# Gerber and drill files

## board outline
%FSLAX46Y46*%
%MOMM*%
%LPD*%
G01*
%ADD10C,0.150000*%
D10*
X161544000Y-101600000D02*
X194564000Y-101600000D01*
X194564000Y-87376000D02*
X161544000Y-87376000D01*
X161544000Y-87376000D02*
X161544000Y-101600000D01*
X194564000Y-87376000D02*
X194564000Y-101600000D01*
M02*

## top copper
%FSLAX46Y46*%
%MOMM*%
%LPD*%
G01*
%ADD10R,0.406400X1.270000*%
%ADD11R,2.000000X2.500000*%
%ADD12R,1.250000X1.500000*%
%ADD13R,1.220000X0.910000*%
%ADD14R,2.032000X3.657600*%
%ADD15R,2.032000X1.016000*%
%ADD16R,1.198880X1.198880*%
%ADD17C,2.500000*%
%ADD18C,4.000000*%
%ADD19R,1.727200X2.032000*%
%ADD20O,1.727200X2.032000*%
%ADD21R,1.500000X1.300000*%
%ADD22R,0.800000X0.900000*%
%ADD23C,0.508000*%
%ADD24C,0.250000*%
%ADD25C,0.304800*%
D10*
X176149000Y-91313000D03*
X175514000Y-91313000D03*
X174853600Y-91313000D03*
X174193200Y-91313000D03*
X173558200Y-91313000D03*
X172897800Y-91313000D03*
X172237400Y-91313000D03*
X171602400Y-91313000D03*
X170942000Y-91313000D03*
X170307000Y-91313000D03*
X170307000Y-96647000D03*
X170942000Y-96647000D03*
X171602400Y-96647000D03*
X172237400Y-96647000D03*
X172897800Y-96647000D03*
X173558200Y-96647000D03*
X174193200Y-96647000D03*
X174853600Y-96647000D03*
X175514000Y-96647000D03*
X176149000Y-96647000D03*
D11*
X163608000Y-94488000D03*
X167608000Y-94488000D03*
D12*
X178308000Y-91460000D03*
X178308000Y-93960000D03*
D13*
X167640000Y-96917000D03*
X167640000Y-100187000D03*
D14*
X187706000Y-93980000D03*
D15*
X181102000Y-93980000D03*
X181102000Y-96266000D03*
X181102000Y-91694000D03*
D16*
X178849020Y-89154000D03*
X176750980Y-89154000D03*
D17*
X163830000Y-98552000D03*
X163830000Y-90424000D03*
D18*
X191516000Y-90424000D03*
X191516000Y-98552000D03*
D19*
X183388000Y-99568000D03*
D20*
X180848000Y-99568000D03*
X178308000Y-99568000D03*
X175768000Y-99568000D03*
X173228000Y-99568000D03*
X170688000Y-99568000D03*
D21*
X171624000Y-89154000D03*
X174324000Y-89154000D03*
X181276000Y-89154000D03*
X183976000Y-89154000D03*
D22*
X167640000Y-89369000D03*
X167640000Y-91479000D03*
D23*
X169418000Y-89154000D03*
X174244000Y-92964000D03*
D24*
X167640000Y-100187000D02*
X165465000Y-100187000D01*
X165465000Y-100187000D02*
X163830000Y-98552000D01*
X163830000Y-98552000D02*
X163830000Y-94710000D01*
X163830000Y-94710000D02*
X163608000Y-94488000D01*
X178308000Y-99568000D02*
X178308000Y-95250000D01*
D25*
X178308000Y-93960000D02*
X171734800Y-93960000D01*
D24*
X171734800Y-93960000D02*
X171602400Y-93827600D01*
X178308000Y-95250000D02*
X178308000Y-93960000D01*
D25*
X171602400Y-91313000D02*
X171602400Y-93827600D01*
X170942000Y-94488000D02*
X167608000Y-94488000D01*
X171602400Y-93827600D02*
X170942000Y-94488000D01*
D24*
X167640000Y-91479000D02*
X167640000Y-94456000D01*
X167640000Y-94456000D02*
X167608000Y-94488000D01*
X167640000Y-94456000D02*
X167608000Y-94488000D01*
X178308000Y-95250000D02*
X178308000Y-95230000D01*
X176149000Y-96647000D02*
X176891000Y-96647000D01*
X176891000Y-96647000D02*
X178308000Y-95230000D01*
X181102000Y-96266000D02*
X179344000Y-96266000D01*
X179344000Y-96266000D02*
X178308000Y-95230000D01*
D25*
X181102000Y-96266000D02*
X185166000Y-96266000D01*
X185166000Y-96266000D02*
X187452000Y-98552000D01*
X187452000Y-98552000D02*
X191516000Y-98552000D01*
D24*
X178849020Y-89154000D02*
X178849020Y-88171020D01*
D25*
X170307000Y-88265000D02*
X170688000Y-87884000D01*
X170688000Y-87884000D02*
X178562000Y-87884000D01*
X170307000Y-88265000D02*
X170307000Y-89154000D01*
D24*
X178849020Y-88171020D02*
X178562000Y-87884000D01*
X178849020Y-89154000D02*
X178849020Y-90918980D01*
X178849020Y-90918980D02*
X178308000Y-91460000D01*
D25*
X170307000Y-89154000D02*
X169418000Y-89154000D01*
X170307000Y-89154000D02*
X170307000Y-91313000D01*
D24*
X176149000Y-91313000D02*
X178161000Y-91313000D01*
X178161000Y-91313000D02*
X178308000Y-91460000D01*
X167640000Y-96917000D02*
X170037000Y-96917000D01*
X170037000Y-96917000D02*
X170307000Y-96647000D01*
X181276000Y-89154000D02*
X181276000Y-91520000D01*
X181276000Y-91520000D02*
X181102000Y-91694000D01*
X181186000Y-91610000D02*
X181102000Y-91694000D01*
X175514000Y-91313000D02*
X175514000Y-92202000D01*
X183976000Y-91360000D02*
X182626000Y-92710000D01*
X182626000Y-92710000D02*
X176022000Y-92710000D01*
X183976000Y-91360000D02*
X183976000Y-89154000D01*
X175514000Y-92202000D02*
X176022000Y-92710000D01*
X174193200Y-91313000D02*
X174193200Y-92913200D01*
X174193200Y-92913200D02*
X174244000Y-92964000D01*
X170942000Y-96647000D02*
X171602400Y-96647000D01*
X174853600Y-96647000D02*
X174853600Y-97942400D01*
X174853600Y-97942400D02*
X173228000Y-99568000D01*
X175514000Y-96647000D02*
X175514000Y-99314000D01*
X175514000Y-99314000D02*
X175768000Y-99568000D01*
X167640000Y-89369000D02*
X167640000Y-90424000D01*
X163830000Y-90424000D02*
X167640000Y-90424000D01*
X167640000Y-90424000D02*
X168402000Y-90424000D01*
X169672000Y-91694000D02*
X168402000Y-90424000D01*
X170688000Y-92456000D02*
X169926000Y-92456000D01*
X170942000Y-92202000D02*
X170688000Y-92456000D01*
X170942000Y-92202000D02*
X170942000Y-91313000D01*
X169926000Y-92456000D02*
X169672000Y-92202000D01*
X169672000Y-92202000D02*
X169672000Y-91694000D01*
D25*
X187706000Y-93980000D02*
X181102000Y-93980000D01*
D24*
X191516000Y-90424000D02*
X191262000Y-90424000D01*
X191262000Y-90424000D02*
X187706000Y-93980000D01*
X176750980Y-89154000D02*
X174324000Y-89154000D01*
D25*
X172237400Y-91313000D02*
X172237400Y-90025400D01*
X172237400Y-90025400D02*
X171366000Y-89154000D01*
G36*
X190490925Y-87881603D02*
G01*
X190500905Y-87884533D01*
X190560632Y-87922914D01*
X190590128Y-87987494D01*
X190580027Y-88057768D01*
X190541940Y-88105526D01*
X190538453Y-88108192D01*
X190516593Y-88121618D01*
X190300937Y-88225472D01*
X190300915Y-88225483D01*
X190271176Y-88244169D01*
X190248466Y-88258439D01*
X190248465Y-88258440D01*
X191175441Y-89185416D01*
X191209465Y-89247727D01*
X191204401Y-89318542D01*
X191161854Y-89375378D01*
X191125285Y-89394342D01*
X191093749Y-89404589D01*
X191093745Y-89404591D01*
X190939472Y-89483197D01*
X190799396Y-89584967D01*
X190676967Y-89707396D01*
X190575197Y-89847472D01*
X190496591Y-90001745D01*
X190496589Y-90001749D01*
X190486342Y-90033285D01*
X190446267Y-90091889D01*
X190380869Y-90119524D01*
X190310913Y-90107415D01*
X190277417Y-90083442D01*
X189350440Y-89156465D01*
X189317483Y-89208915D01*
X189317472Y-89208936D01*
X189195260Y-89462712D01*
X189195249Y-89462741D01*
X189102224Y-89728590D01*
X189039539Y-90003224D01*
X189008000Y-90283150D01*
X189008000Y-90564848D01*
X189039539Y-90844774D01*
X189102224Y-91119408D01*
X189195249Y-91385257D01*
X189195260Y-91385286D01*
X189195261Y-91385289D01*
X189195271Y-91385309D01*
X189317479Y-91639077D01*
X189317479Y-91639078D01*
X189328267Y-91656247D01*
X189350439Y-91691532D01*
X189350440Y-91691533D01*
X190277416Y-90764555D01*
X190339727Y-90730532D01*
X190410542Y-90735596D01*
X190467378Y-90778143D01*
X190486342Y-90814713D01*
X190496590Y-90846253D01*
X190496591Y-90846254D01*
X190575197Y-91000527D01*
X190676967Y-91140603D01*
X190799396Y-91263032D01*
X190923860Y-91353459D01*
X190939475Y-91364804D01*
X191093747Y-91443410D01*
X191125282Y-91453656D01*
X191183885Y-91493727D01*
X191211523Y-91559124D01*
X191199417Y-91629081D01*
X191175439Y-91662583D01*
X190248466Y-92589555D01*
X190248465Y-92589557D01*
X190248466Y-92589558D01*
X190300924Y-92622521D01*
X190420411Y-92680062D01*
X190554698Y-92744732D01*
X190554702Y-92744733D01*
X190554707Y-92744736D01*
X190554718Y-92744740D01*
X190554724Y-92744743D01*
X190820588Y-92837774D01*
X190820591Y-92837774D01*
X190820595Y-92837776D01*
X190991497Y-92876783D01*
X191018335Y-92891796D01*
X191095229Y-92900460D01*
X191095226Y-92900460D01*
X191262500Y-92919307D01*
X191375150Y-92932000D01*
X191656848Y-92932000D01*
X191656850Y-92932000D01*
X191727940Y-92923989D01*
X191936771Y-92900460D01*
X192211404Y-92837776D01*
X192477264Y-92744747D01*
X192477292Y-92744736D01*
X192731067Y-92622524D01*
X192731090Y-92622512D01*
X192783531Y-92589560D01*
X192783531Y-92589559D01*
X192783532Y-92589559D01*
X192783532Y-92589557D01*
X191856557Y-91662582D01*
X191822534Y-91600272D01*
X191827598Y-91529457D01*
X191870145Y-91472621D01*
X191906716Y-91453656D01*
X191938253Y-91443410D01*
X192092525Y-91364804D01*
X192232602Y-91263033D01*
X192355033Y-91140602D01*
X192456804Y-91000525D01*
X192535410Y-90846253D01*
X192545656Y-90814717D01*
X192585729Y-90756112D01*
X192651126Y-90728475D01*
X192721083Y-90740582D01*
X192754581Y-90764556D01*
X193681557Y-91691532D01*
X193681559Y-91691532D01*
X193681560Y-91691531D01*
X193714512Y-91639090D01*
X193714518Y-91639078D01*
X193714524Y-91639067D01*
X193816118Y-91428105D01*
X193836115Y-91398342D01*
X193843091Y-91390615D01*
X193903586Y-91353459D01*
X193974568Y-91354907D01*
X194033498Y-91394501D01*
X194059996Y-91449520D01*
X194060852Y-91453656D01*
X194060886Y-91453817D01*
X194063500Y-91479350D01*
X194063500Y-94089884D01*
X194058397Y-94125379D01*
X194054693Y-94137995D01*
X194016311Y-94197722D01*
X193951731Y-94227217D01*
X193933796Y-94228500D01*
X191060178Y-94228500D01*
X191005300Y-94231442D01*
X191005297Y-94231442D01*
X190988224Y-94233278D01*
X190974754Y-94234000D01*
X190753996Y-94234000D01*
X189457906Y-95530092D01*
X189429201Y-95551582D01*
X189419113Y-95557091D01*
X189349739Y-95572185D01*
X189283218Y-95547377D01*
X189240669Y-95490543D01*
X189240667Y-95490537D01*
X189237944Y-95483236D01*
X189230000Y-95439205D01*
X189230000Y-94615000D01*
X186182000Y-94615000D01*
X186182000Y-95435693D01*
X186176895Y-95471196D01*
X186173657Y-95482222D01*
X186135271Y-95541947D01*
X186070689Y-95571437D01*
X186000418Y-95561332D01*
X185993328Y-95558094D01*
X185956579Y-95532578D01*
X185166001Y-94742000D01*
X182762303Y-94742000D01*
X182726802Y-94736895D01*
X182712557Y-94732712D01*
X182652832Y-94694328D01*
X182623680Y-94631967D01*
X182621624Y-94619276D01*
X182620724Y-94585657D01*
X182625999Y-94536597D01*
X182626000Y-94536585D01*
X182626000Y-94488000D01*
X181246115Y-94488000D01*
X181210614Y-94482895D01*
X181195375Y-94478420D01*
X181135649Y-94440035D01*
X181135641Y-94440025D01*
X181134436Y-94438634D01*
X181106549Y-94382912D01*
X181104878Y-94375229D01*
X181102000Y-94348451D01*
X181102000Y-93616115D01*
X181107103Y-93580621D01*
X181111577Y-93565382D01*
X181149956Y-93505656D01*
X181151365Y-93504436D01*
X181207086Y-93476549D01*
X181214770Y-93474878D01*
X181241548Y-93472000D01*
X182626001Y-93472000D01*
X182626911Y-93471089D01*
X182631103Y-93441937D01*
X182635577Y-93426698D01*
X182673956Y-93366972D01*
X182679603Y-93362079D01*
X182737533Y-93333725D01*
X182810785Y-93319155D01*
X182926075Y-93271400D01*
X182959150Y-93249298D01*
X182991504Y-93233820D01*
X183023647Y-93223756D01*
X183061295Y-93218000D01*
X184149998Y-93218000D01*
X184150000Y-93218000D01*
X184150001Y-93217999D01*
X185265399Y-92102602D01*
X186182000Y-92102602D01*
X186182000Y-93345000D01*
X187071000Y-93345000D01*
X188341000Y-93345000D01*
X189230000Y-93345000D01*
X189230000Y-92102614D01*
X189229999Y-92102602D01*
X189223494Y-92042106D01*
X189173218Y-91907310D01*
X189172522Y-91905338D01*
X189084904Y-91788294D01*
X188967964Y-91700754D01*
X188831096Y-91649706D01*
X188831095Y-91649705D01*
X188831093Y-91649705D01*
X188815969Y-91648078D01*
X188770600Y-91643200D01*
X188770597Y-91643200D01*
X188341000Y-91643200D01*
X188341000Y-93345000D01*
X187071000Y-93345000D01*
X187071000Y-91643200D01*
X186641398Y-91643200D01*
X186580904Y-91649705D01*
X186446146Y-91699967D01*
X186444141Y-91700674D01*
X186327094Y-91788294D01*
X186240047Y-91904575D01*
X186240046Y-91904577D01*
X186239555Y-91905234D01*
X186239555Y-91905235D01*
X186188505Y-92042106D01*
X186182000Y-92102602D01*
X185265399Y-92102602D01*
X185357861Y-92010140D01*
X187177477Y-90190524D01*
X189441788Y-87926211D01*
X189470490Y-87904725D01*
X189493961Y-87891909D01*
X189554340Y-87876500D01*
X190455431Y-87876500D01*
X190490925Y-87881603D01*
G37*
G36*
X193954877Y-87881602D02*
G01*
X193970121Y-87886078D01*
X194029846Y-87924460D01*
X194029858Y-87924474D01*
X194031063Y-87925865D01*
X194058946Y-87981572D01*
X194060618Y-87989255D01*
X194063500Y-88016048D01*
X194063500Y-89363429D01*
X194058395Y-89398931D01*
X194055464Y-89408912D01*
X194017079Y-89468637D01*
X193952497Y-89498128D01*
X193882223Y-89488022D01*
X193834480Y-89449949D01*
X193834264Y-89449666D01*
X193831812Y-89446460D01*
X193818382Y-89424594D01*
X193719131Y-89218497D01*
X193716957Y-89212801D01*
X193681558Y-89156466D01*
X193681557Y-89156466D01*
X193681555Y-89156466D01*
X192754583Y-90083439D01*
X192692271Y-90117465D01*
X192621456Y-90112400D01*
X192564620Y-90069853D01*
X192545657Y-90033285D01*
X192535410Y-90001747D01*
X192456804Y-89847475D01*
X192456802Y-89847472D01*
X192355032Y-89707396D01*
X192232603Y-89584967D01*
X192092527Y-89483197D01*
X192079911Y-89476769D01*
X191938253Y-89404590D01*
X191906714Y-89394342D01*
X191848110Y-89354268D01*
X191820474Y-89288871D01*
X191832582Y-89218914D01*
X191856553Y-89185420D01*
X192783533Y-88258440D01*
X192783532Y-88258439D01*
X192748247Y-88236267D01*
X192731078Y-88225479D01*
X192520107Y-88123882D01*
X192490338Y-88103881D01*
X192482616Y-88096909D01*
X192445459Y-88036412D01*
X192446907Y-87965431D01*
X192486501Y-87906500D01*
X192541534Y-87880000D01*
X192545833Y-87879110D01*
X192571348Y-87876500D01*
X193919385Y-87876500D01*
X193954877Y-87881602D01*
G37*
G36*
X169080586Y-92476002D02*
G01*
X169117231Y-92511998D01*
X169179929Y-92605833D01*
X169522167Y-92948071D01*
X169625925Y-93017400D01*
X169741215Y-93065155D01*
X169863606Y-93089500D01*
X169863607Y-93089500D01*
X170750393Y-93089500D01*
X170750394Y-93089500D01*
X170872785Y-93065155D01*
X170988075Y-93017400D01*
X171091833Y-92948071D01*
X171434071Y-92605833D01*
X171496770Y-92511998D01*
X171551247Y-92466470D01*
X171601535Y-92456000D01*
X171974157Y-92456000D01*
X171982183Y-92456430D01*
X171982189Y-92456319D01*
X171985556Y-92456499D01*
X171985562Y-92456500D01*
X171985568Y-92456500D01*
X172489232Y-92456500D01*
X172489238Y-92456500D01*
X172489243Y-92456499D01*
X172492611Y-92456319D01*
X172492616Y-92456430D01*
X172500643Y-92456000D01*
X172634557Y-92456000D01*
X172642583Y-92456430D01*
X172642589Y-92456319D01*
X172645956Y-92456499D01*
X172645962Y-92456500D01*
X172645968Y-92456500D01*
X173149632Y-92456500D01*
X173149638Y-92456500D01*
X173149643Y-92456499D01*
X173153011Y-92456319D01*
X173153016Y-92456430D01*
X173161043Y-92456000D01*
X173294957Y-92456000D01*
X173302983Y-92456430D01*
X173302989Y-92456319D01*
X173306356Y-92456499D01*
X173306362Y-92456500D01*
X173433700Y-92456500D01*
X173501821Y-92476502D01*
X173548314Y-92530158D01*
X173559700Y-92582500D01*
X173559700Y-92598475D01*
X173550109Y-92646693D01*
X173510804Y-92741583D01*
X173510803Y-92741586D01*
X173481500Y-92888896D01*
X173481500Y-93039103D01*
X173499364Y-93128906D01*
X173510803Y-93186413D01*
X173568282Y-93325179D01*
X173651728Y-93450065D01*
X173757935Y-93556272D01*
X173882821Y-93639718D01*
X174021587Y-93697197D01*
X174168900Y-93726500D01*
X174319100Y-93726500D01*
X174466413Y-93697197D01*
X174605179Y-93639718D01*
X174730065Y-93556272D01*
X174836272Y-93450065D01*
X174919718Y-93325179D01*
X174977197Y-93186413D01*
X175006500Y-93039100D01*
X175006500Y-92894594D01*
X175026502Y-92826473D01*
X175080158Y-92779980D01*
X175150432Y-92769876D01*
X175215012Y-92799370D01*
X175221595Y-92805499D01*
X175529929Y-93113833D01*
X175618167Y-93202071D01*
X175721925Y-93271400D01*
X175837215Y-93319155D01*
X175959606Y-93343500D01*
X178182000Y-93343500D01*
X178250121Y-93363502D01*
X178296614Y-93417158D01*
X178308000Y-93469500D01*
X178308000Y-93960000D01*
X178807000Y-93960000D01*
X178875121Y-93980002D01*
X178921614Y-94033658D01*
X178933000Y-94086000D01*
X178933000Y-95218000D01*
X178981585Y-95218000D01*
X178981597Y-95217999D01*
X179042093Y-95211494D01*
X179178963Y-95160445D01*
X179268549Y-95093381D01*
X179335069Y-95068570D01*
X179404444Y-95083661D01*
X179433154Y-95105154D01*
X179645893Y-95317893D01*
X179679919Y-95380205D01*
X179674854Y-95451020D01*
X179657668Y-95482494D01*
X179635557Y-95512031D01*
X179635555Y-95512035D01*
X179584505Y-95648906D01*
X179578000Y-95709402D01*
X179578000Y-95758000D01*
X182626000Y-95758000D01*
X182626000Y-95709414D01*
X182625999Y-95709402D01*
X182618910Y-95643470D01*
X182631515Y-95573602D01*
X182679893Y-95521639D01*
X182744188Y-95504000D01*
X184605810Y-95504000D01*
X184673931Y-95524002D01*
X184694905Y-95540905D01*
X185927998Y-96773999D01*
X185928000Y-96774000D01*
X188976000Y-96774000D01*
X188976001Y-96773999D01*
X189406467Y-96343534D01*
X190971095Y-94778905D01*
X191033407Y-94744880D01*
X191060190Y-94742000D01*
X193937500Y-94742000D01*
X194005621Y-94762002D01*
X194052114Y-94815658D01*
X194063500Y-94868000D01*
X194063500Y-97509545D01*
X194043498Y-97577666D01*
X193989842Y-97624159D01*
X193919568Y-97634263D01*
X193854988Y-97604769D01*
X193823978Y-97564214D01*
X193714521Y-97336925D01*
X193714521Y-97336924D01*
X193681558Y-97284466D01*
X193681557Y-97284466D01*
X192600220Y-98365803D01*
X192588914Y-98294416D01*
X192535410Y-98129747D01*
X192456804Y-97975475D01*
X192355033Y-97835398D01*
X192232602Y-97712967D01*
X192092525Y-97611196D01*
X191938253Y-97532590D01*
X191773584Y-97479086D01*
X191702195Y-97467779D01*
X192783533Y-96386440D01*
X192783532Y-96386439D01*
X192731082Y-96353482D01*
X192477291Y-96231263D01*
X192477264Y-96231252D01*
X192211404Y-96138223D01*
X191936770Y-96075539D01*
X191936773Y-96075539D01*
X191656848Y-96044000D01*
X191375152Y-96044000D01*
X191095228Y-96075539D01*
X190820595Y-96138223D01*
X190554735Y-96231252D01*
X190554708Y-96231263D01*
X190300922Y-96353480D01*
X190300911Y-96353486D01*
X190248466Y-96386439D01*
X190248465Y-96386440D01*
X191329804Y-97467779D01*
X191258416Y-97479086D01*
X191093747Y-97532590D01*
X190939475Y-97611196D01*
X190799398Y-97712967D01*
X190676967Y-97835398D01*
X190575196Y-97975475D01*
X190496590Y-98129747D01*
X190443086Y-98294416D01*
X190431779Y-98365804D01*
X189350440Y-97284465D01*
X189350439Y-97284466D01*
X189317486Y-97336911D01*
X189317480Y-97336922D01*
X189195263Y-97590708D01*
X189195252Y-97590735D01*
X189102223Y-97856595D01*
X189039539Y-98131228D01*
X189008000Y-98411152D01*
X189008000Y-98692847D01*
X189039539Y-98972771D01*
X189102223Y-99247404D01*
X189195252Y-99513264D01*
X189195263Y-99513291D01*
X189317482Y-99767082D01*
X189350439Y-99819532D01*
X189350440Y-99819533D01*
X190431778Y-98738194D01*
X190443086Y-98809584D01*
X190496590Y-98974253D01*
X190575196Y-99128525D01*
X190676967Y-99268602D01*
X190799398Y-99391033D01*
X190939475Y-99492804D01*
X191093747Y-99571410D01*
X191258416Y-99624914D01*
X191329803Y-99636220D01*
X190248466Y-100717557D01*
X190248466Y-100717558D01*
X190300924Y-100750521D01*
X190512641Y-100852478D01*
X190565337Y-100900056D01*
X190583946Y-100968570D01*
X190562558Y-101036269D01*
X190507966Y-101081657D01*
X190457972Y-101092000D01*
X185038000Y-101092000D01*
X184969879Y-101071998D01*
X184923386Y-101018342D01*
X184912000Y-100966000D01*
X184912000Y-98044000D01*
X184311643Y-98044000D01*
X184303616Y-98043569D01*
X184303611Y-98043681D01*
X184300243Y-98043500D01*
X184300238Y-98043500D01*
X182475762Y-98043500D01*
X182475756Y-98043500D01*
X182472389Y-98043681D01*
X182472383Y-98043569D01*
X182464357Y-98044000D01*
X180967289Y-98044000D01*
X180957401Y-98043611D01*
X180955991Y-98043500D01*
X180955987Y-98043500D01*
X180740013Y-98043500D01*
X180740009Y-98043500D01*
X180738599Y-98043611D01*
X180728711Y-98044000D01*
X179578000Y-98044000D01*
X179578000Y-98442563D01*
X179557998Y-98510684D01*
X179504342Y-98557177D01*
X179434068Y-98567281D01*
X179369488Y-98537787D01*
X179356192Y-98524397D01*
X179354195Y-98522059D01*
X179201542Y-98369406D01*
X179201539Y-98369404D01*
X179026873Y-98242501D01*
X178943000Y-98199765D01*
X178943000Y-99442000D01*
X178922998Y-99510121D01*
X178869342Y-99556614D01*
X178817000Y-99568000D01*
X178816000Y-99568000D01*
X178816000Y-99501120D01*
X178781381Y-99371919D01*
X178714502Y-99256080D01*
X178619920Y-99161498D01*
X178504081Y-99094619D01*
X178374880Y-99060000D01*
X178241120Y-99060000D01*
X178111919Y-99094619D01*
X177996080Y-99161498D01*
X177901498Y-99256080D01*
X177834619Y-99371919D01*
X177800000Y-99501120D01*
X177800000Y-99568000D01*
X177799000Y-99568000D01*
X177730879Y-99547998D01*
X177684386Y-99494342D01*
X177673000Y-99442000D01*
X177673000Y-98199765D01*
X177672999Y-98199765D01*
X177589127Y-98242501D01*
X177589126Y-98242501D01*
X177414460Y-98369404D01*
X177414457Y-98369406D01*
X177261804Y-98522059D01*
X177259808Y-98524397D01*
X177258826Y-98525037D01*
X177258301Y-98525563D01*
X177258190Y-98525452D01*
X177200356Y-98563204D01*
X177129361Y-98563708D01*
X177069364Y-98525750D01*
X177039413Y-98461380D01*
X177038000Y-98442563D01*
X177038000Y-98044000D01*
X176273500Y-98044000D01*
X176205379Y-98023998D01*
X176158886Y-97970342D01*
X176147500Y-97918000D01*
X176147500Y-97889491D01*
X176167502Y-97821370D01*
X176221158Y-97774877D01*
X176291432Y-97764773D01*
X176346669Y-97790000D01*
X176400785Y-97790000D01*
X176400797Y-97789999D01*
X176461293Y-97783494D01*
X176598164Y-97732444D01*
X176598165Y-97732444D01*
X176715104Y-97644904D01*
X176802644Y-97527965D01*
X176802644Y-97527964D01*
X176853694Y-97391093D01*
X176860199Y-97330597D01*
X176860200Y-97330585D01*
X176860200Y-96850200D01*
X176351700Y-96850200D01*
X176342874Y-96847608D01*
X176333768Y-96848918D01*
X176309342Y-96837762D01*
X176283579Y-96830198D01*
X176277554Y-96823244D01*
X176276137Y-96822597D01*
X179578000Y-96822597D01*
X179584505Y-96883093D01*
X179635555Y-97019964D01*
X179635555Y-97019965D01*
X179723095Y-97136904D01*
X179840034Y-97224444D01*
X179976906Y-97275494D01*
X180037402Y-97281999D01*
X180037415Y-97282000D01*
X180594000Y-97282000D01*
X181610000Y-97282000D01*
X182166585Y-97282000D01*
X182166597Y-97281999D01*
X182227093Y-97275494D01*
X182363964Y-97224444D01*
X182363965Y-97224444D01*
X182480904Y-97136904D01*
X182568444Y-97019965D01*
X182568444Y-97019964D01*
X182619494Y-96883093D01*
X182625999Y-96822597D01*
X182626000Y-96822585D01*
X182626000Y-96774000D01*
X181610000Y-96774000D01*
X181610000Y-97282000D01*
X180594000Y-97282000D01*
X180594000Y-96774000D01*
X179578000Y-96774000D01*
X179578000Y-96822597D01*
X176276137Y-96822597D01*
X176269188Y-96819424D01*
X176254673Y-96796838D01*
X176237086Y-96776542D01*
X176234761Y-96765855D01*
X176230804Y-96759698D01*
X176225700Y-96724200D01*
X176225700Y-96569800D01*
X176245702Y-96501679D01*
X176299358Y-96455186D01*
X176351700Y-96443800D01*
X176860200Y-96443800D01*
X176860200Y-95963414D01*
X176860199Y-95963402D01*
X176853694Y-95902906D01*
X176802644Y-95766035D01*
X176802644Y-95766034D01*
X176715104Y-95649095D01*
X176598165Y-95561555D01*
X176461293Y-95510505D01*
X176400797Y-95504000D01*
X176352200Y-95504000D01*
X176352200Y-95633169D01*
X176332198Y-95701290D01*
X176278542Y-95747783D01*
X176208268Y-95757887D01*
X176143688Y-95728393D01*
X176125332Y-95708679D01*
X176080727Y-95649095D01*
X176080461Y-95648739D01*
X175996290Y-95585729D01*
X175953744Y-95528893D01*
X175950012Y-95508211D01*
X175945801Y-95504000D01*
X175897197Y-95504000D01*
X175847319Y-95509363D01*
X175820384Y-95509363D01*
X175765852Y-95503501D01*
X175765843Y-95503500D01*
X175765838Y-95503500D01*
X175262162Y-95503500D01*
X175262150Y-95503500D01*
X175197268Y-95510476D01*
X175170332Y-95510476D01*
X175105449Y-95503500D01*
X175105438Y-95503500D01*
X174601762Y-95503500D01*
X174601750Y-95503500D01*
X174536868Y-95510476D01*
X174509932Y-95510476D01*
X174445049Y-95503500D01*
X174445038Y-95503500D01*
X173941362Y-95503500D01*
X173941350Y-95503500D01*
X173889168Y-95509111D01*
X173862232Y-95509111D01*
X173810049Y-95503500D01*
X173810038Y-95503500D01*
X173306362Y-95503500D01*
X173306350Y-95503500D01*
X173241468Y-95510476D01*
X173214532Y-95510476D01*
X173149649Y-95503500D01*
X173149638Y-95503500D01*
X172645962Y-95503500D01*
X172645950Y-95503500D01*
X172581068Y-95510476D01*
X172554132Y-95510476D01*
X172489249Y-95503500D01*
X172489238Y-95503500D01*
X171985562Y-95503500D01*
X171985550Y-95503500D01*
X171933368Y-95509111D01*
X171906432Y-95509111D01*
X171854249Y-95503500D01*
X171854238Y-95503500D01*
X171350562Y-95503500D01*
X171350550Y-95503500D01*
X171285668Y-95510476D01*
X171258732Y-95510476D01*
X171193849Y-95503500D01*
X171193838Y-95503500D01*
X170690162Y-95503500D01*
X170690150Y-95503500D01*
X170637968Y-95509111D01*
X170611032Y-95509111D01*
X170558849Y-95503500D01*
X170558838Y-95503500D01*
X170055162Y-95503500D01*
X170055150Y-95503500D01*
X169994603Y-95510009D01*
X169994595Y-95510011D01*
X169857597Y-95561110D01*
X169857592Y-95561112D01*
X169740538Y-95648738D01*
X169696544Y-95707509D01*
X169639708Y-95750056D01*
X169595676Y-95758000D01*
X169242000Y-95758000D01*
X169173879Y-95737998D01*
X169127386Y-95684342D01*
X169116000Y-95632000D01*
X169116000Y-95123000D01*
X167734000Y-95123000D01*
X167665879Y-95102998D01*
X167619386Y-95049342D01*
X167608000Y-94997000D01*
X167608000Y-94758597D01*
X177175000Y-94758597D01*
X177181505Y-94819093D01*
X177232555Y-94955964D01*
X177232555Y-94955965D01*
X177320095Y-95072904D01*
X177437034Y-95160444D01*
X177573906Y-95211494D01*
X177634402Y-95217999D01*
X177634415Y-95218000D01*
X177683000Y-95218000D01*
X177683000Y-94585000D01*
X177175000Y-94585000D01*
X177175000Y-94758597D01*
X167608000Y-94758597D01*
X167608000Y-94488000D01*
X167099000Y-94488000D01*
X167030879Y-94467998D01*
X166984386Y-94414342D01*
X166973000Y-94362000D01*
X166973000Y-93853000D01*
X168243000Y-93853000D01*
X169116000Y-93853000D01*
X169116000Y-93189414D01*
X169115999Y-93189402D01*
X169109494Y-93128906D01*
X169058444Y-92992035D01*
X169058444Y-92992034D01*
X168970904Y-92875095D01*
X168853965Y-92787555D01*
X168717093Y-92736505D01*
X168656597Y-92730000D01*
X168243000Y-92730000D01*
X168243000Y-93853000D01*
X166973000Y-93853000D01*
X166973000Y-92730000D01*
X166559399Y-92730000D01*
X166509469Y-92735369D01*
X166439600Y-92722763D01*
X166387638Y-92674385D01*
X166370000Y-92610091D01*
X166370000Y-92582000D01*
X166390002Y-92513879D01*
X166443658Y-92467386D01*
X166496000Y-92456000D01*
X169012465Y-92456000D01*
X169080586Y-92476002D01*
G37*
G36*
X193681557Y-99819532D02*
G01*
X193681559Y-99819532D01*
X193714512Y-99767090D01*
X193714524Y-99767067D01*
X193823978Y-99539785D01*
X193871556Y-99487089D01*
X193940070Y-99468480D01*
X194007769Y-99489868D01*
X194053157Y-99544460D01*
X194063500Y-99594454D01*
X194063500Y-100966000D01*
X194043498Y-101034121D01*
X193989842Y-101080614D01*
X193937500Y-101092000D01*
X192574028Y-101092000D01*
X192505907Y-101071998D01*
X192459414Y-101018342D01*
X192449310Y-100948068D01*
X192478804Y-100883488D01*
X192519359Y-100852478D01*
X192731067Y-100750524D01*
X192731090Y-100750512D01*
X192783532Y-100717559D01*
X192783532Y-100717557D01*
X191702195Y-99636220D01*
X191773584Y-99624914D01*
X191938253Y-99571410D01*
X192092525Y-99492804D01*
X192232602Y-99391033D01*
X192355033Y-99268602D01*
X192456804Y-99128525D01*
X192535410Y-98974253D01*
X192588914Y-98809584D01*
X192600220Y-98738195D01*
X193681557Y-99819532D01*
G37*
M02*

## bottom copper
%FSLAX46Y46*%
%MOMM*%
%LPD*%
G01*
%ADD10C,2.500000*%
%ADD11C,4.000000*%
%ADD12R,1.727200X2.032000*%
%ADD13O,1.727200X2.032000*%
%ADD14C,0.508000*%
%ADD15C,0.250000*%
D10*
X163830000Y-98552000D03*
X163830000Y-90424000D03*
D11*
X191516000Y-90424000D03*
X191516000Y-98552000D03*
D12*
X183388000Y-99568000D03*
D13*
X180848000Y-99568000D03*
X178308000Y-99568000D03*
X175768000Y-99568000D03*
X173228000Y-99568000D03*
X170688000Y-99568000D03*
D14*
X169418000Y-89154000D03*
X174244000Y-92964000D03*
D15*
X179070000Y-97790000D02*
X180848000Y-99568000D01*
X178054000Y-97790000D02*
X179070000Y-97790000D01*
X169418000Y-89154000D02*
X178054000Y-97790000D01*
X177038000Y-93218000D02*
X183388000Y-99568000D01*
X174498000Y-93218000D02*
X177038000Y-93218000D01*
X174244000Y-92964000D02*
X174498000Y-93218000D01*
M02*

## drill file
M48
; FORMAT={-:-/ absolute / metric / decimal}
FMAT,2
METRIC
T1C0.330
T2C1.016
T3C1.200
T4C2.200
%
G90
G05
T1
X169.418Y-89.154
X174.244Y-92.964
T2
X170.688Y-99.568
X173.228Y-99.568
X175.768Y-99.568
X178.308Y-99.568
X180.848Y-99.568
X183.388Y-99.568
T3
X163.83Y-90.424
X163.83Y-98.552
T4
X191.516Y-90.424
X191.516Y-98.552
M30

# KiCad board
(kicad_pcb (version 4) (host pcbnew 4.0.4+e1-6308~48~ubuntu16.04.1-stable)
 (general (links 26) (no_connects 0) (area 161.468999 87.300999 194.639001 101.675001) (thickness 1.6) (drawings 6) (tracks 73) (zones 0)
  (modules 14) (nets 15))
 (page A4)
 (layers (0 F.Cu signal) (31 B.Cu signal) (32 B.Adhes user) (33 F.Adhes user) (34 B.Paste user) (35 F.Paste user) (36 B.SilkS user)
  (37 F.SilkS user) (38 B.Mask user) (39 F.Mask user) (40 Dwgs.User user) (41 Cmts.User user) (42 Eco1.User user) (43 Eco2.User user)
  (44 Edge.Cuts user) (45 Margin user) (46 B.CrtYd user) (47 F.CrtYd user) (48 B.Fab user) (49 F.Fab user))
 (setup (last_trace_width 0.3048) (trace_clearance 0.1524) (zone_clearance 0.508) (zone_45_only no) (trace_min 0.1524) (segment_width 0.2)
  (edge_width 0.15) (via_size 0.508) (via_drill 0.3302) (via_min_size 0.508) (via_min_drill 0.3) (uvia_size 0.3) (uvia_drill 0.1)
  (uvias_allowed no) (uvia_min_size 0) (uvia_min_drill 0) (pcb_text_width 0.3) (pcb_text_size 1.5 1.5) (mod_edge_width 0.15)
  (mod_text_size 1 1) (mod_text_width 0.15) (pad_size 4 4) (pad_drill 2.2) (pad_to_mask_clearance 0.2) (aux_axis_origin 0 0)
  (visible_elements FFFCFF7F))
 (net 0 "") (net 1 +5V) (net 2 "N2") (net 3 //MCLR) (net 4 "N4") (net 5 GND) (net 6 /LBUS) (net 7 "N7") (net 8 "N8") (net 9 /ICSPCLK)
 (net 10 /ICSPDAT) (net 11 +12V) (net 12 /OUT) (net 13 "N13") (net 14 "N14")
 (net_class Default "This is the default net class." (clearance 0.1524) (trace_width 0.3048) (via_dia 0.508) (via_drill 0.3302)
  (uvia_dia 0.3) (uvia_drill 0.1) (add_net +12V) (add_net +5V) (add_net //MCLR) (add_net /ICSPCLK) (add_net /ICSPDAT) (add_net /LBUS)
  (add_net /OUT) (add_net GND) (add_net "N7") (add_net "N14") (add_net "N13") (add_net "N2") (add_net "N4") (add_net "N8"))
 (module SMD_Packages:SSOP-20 (layer F.Cu) (at 173.228 93.98 180)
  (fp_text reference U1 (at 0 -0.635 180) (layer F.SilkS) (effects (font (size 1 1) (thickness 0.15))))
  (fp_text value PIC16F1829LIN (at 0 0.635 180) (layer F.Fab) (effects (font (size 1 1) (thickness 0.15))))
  (pad 1 smd rect (at -2.921 2.667 180) (size 0.4064 1.27) (layers F.Cu F.Paste F.Mask) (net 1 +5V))
  (pad 2 smd rect (at -2.286 2.667 180) (size 0.4064 1.27) (layers F.Cu F.Paste F.Mask) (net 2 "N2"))
  (pad 3 smd rect (at -1.6256 2.667 180) (size 0.4064 1.27) (layers F.Cu F.Paste F.Mask))
  (pad 4 smd rect (at -0.9652 2.667 180) (size 0.4064 1.27) (layers F.Cu F.Paste F.Mask) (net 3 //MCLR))
  (pad 5 smd rect (at -0.3302 2.667 180) (size 0.4064 1.27) (layers F.Cu F.Paste F.Mask))
  (pad 6 smd rect (at 0.3302 2.667 180) (size 0.4064 1.27) (layers F.Cu F.Paste F.Mask))
  (pad 7 smd rect (at 0.9906 2.667 180) (size 0.4064 1.27) (layers F.Cu F.Paste F.Mask) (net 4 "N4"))
  (pad 8 smd rect (at 1.6256 2.667 180) (size 0.4064 1.27) (layers F.Cu F.Paste F.Mask) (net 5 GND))
  (pad 9 smd rect (at 2.286 2.667 180) (size 0.4064 1.27) (layers F.Cu F.Paste F.Mask) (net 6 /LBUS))
  (pad 10 smd rect (at 2.921 2.667 180) (size 0.4064 1.27) (layers F.Cu F.Paste F.Mask) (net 1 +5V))
  (pad 11 smd rect (at 2.921 -2.667 180) (size 0.4064 1.27) (layers F.Cu F.Paste F.Mask) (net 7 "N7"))
  (pad 12 smd rect (at 2.286 -2.667 180) (size 0.4064 1.27) (layers F.Cu F.Paste F.Mask) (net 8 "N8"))
  (pad 13 smd rect (at 1.6256 -2.667 180) (size 0.4064 1.27) (layers F.Cu F.Paste F.Mask) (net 8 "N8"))
  (pad 14 smd rect (at 0.9906 -2.667 180) (size 0.4064 1.27) (layers F.Cu F.Paste F.Mask))
  (pad 15 smd rect (at 0.3302 -2.667 180) (size 0.4064 1.27) (layers F.Cu F.Paste F.Mask))
  (pad 16 smd rect (at -0.3302 -2.667 180) (size 0.4064 1.27) (layers F.Cu F.Paste F.Mask))
  (pad 17 smd rect (at -0.9652 -2.667 180) (size 0.4064 1.27) (layers F.Cu F.Paste F.Mask))
  (pad 18 smd rect (at -1.6256 -2.667 180) (size 0.4064 1.27) (layers F.Cu F.Paste F.Mask) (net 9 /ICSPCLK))
  (pad 19 smd rect (at -2.286 -2.667 180) (size 0.4064 1.27) (layers F.Cu F.Paste F.Mask) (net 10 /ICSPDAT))
  (pad 20 smd rect (at -2.921 -2.667 180) (size 0.4064 1.27) (layers F.Cu F.Paste F.Mask) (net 5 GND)))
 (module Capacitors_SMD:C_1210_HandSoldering (layer F.Cu) (at 165.608 94.488)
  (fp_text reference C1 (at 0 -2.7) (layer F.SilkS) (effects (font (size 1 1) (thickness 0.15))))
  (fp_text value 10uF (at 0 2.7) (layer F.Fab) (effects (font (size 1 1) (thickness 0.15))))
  (pad 1 smd rect (at -2 0) (size 2 2.5) (layers F.Cu F.Paste F.Mask) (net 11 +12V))
  (pad 2 smd rect (at 2 0) (size 2 2.5) (layers F.Cu F.Paste F.Mask) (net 5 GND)))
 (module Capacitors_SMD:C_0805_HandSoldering (layer F.Cu) (at 178.308 92.71 270)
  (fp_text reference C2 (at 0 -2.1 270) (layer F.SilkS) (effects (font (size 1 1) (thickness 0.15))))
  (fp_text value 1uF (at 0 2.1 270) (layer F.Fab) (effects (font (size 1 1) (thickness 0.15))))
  (pad 1 smd rect (at -1.25 0 270) (size 1.5 1.25) (layers F.Cu F.Paste F.Mask) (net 1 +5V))
  (pad 2 smd rect (at 1.25 0 270) (size 1.5 1.25) (layers F.Cu F.Paste F.Mask) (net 5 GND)))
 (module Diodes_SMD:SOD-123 (layer F.Cu) (at 167.64 98.552 270)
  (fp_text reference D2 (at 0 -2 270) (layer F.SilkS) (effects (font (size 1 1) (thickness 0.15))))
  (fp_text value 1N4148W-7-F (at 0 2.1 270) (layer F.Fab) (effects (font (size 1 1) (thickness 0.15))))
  (pad 1 smd rect (at -1.635 0 270) (size 0.91 1.22) (layers F.Cu F.Paste F.Mask) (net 7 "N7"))
  (pad 2 smd rect (at 1.635 0 270) (size 0.91 1.22) (layers F.Cu F.Paste F.Mask) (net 11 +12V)))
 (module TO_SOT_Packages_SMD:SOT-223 (layer F.Cu) (at 184.404 93.98 270)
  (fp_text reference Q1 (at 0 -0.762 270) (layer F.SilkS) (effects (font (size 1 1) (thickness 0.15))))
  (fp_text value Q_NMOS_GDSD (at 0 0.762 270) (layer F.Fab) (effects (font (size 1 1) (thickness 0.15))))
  (pad 4 smd rect (at 0 -3.302 270) (size 3.6576 2.032) (layers F.Cu F.Paste F.Mask) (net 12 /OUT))
  (pad 2 smd rect (at 0 3.302 270) (size 1.016 2.032) (layers F.Cu F.Paste F.Mask) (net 12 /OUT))
  (pad 3 smd rect (at 2.286 3.302 270) (size 1.016 2.032) (layers F.Cu F.Paste F.Mask) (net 5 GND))
  (pad 1 smd rect (at -2.286 3.302 270) (size 1.016 2.032) (layers F.Cu F.Paste F.Mask) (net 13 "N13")))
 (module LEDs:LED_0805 (layer F.Cu) (at 177.8 89.154)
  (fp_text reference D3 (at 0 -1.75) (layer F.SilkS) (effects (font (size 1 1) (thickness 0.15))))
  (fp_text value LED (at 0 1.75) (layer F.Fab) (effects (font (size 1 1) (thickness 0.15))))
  (pad 2 smd rect (at 1.04902 0 180) (size 1.19888 1.19888) (layers F.Cu F.Paste F.Mask) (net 1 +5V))
  (pad 1 smd rect (at -1.04902 0 180) (size 1.19888 1.19888) (layers F.Cu F.Paste F.Mask) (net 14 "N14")))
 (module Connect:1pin (layer F.Cu) (at 163.83 98.552)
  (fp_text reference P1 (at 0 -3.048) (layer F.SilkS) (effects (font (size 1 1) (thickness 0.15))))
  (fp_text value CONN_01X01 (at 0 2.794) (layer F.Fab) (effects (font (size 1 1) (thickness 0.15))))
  (pad 1 thru_hole circle (at 0 0) (size 2.5 2.5) (drill 1.2) (layers *.Cu *.Mask F.SilkS) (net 11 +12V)))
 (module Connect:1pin (layer F.Cu) (at 163.83 90.424)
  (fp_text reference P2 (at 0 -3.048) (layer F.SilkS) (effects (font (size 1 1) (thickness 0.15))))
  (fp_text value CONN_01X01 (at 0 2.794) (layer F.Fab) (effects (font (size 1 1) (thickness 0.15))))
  (pad 1 thru_hole circle (at 0 0) (size 2.5 2.5) (drill 1.2) (layers *.Cu *.Mask F.SilkS) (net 6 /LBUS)))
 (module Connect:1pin (layer F.Cu) (at 191.516 90.424)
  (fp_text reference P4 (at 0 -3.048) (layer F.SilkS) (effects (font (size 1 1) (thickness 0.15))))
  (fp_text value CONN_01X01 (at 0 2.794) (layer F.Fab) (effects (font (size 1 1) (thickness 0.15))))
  (pad 1 thru_hole circle (at 0 0) (size 4 4) (drill 2.2) (layers *.Cu *.Mask F.SilkS) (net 12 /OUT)))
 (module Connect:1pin (layer F.Cu) (at 191.516 98.552)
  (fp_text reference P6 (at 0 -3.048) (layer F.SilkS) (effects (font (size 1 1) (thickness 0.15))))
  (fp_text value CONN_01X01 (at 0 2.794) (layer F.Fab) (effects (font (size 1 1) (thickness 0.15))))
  (pad 1 thru_hole circle (at 0 0) (size 4 4) (drill 2.2) (layers *.Cu *.Mask F.SilkS) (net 5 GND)))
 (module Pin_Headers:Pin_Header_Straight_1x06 (layer F.Cu) (at 183.388 99.568 270)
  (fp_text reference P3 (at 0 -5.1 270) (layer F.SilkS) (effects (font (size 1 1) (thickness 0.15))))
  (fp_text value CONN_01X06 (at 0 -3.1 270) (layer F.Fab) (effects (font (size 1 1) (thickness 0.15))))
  (pad 1 thru_hole rect (at 0 0 270) (size 2.032 1.7272) (drill 1.016) (layers *.Cu *.Mask F.SilkS) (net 3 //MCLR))
  (pad 2 thru_hole oval (at 0 2.54 270) (size 2.032 1.7272) (drill 1.016) (layers *.Cu *.Mask F.SilkS) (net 1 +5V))
  (pad 3 thru_hole oval (at 0 5.08 270) (size 2.032 1.7272) (drill 1.016) (layers *.Cu *.Mask F.SilkS) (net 5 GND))
  (pad 4 thru_hole oval (at 0 7.62 270) (size 2.032 1.7272) (drill 1.016) (layers *.Cu *.Mask F.SilkS) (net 10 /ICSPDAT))
  (pad 5 thru_hole oval (at 0 10.16 270) (size 2.032 1.7272) (drill 1.016) (layers *.Cu *.Mask F.SilkS) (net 9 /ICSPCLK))
  (pad 6 thru_hole oval (at 0 12.7 270) (size 2.032 1.7272) (drill 1.016) (layers *.Cu *.Mask F.SilkS)))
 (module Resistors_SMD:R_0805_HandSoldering (layer F.Cu) (at 172.974 89.154)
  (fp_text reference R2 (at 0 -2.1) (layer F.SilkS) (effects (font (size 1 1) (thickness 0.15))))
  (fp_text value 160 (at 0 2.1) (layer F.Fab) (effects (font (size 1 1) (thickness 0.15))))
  (pad 1 smd rect (at -1.35 0) (size 1.5 1.3) (layers F.Cu F.Paste F.Mask) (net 4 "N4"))
  (pad 2 smd rect (at 1.35 0) (size 1.5 1.3) (layers F.Cu F.Paste F.Mask) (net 14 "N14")))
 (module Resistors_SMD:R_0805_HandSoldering (layer F.Cu) (at 182.626 89.154)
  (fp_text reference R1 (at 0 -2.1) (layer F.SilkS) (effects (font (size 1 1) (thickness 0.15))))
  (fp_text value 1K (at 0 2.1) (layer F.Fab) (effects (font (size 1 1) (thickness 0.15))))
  (pad 1 smd rect (at -1.35 0) (size 1.5 1.3) (layers F.Cu F.Paste F.Mask) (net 13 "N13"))
  (pad 2 smd rect (at 1.35 0) (size 1.5 1.3) (layers F.Cu F.Paste F.Mask) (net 2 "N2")))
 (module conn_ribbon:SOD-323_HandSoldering (layer F.Cu) (at 167.64 90.424 270)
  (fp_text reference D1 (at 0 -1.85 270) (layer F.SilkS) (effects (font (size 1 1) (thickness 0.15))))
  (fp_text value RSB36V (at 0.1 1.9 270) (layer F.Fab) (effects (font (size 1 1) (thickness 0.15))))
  (pad 1 smd rect (at -1.055 0 270) (size 0.9 0.8) (layers F.Cu F.Paste F.Mask) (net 6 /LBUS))
  (pad 2 smd rect (at 1.055 0 270) (size 0.9 0.8) (layers F.Cu F.Paste F.Mask) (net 5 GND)))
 (gr_line (start 161.544 101.6) (end 194.564 101.6) (angle 90) (layer Edge.Cuts) (width 0.15))
 (gr_line (start 194.564 87.376) (end 161.544 87.376) (angle 90) (layer Edge.Cuts) (width 0.15))
 (gr_line (start 161.544 87.376) (end 161.544 101.6) (angle 90) (layer Edge.Cuts) (width 0.15))
 (gr_line (start 194.564 87.376) (end 194.564 101.6) (angle 90) (layer Edge.Cuts) (width 0.15))
 (segment (start 167.64 100.187) (end 165.465 100.187) (width 0.25) (layer F.Cu) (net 11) (status 10))
 (segment (start 165.465 100.187) (end 163.83 98.552) (width 0.25) (layer F.Cu) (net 11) (status 20))
 (segment (start 163.83 98.552) (end 163.83 94.71) (width 0.25) (layer F.Cu) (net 11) (status 30))
 (segment (start 163.83 94.71) (end 163.608 94.488) (width 0.25) (layer F.Cu) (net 11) (status 30))
 (segment (start 178.308 99.568) (end 178.308 95.25) (width 0.25) (layer F.Cu) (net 5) (status 10))
 (segment (start 178.308 93.96) (end 171.7348 93.96) (width 0.3048) (layer F.Cu) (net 5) (status 10))
 (segment (start 171.7348 93.96) (end 171.6024 93.8276) (width 0.25) (layer F.Cu) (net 5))
 (segment (start 178.308 95.25) (end 178.308 93.96) (width 0.25) (layer F.Cu) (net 5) (status 20))
 (segment (start 171.6024 91.313) (end 171.6024 93.8276) (width 0.3048) (layer F.Cu) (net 5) (status 10))
 (segment (start 170.942 94.488) (end 167.608 94.488) (width 0.3048) (layer F.Cu) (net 5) (status 20))
 (segment (start 171.6024 93.8276) (end 170.942 94.488) (width 0.3048) (layer F.Cu) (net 5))
 (segment (start 167.64 91.479) (end 167.64 94.456) (width 0.25) (layer F.Cu) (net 5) (status 30))
 (segment (start 167.64 94.456) (end 167.608 94.488) (width 0.25) (layer F.Cu) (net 5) (status 30))
 (segment (start 167.64 94.456) (end 167.608 94.488) (width 0.25) (layer F.Cu) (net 5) (status 30))
 (segment (start 178.308 95.25) (end 178.308 95.23) (width 0.25) (layer F.Cu) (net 5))
 (segment (start 176.149 96.647) (end 176.891 96.647) (width 0.25) (layer F.Cu) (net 5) (status 10))
 (segment (start 176.891 96.647) (end 178.308 95.23) (width 0.25) (layer F.Cu) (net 5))
 (segment (start 181.102 96.266) (end 179.344 96.266) (width 0.25) (layer F.Cu) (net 5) (status 10))
 (segment (start 179.344 96.266) (end 178.308 95.23) (width 0.25) (layer F.Cu) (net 5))
 (segment (start 181.102 96.266) (end 185.166 96.266) (width 0.3048) (layer F.Cu) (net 5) (status 10))
 (segment (start 185.166 96.266) (end 187.452 98.552) (width 0.3048) (layer F.Cu) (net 5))
 (segment (start 187.452 98.552) (end 191.516 98.552) (width 0.3048) (layer F.Cu) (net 5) (status 20))
 (segment (start 178.84902 89.154) (end 178.84902 88.17102) (width 0.25) (layer F.Cu) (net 1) (status 10))
 (segment (start 170.307 88.265) (end 170.688 87.884) (width 0.3048) (layer F.Cu) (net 1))
 (segment (start 170.688 87.884) (end 178.562 87.884) (width 0.3048) (layer F.Cu) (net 1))
 (segment (start 170.307 88.265) (end 170.307 89.154) (width 0.3048) (layer F.Cu) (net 1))
 (segment (start 178.84902 88.17102) (end 178.562 87.884) (width 0.25) (layer F.Cu) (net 1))
 (segment (start 178.84902 89.154) (end 178.84902 90.91898) (width 0.25) (layer F.Cu) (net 1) (status 30))
 (segment (start 178.84902 90.91898) (end 178.308 91.46) (width 0.25) (layer F.Cu) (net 1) (status 30))
 (segment (start 170.307 89.154) (end 169.418 89.154) (width 0.3048) (layer F.Cu) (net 1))
 (segment (start 179.07 97.79) (end 180.848 99.568) (width 0.25) (layer B.Cu) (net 1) (status 20))
 (segment (start 178.054 97.79) (end 179.07 97.79) (width 0.25) (layer B.Cu) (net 1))
 (segment (start 169.418 89.154) (end 178.054 97.79) (width 0.25) (layer B.Cu) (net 1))
 (via (at 169.418 89.154) (size 0.508) (drill 0.3302) (layers F.Cu B.Cu) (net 1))
 (segment (start 170.307 89.154) (end 170.307 91.313) (width 0.3048) (layer F.Cu) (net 1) (status 20))
 (segment (start 176.149 91.313) (end 178.161 91.313) (width 0.25) (layer F.Cu) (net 1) (status 30))
 (segment (start 178.161 91.313) (end 178.308 91.46) (width 0.25) (layer F.Cu) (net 1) (status 30))
 (segment (start 167.64 96.917) (end 170.037 96.917) (width 0.25) (layer F.Cu) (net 7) (status 10))
 (segment (start 170.037 96.917) (end 170.307 96.647) (width 0.25) (layer F.Cu) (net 7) (status 20))
 (segment (start 181.276 89.154) (end 181.276 91.52) (width 0.25) (layer F.Cu) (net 13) (status 30))
 (segment (start 181.276 91.52) (end 181.102 91.694) (width 0.25) (layer F.Cu) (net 13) (status 30))
 (segment (start 181.186 91.61) (end 181.102 91.694) (width 0.25) (layer F.Cu) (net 13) (status 30))
 (segment (start 175.514 91.313) (end 175.514 92.202) (width 0.25) (layer F.Cu) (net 2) (status 10))
 (segment (start 183.976 91.36) (end 182.626 92.71) (width 0.25) (layer F.Cu) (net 2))
 (segment (start 182.626 92.71) (end 176.022 92.71) (width 0.25) (layer F.Cu) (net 2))
 (segment (start 183.976 91.36) (end 183.976 89.154) (width 0.25) (layer F.Cu) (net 2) (status 20))
 (segment (start 175.514 92.202) (end 176.022 92.71) (width 0.25) (layer F.Cu) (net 2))
 (segment (start 174.1932 91.313) (end 174.1932 92.9132) (width 0.25) (layer F.Cu) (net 3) (status 10))
 (segment (start 177.038 93.218) (end 183.388 99.568) (width 0.25) (layer B.Cu) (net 3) (status 20))
 (segment (start 174.498 93.218) (end 177.038 93.218) (width 0.25) (layer B.Cu) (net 3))
 (segment (start 174.244 92.964) (end 174.498 93.218) (width 0.25) (layer B.Cu) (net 3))
 (via (at 174.244 92.964) (size 0.508) (drill 0.3302) (layers F.Cu B.Cu) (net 3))
 (segment (start 174.1932 92.9132) (end 174.244 92.964) (width 0.25) (layer F.Cu) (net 3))
 (segment (start 170.942 96.647) (end 171.6024 96.647) (width 0.25) (layer F.Cu) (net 8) (status 30))
 (segment (start 174.8536 96.647) (end 174.8536 97.9424) (width 0.25) (layer F.Cu) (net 9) (status 10))
 (segment (start 174.8536 97.9424) (end 173.228 99.568) (width 0.25) (layer F.Cu) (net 9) (status 20))
 (segment (start 175.514 96.647) (end 175.514 99.314) (width 0.25) (layer F.Cu) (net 10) (status 30))
 (segment (start 175.514 99.314) (end 175.768 99.568) (width 0.25) (layer F.Cu) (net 10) (status 30))
 (segment (start 167.64 89.369) (end 167.64 90.424) (width 0.25) (layer F.Cu) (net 6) (status 10))
 (segment (start 163.83 90.424) (end 167.64 90.424) (width 0.25) (layer F.Cu) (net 6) (status 10))
 (segment (start 167.64 90.424) (end 168.402 90.424) (width 0.25) (layer F.Cu) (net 6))
 (segment (start 169.672 91.694) (end 168.402 90.424) (width 0.25) (layer F.Cu) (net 6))
 (segment (start 170.688 92.456) (end 169.926 92.456) (width 0.25) (layer F.Cu) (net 6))
 (segment (start 170.942 92.202) (end 170.688 92.456) (width 0.25) (layer F.Cu) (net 6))
 (segment (start 170.942 92.202) (end 170.942 91.313) (width 0.25) (layer F.Cu) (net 6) (status 20))
 (segment (start 169.926 92.456) (end 169.672 92.202) (width 0.25) (layer F.Cu) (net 6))
 (segment (start 169.672 92.202) (end 169.672 91.694) (width 0.25) (layer F.Cu) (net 6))
 (segment (start 187.706 93.98) (end 181.102 93.98) (width 0.3048) (layer F.Cu) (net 12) (status 30))
 (segment (start 191.516 90.424) (end 191.262 90.424) (width 0.25) (layer F.Cu) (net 12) (status 30))
 (segment (start 191.262 90.424) (end 187.706 93.98) (width 0.25) (layer F.Cu) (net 12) (status 30))
 (segment (start 176.75098 89.154) (end 174.324 89.154) (width 0.25) (layer F.Cu) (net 14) (status 30))
 (segment (start 172.2374 91.313) (end 172.2374 90.0254) (width 0.3048) (layer F.Cu) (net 4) (status 10))
 (segment (start 172.2374 90.0254) (end 171.366 89.154) (width 0.3048) (layer F.Cu) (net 4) (status 20))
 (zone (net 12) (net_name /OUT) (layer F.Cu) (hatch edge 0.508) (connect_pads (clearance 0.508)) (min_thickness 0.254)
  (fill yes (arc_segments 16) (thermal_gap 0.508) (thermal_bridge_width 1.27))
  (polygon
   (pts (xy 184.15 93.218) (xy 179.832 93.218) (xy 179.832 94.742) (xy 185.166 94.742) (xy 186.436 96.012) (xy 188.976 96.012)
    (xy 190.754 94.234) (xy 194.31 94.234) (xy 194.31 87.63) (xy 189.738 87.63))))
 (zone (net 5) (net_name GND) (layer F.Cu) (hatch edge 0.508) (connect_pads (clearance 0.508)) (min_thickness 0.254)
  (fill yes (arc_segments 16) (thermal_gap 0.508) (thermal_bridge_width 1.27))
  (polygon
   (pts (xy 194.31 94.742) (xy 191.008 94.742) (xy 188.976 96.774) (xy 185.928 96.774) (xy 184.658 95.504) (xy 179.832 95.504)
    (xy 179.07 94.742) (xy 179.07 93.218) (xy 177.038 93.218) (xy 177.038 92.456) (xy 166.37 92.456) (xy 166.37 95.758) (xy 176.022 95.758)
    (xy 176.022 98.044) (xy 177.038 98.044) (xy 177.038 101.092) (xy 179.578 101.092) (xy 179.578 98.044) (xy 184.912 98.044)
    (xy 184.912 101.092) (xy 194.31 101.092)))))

